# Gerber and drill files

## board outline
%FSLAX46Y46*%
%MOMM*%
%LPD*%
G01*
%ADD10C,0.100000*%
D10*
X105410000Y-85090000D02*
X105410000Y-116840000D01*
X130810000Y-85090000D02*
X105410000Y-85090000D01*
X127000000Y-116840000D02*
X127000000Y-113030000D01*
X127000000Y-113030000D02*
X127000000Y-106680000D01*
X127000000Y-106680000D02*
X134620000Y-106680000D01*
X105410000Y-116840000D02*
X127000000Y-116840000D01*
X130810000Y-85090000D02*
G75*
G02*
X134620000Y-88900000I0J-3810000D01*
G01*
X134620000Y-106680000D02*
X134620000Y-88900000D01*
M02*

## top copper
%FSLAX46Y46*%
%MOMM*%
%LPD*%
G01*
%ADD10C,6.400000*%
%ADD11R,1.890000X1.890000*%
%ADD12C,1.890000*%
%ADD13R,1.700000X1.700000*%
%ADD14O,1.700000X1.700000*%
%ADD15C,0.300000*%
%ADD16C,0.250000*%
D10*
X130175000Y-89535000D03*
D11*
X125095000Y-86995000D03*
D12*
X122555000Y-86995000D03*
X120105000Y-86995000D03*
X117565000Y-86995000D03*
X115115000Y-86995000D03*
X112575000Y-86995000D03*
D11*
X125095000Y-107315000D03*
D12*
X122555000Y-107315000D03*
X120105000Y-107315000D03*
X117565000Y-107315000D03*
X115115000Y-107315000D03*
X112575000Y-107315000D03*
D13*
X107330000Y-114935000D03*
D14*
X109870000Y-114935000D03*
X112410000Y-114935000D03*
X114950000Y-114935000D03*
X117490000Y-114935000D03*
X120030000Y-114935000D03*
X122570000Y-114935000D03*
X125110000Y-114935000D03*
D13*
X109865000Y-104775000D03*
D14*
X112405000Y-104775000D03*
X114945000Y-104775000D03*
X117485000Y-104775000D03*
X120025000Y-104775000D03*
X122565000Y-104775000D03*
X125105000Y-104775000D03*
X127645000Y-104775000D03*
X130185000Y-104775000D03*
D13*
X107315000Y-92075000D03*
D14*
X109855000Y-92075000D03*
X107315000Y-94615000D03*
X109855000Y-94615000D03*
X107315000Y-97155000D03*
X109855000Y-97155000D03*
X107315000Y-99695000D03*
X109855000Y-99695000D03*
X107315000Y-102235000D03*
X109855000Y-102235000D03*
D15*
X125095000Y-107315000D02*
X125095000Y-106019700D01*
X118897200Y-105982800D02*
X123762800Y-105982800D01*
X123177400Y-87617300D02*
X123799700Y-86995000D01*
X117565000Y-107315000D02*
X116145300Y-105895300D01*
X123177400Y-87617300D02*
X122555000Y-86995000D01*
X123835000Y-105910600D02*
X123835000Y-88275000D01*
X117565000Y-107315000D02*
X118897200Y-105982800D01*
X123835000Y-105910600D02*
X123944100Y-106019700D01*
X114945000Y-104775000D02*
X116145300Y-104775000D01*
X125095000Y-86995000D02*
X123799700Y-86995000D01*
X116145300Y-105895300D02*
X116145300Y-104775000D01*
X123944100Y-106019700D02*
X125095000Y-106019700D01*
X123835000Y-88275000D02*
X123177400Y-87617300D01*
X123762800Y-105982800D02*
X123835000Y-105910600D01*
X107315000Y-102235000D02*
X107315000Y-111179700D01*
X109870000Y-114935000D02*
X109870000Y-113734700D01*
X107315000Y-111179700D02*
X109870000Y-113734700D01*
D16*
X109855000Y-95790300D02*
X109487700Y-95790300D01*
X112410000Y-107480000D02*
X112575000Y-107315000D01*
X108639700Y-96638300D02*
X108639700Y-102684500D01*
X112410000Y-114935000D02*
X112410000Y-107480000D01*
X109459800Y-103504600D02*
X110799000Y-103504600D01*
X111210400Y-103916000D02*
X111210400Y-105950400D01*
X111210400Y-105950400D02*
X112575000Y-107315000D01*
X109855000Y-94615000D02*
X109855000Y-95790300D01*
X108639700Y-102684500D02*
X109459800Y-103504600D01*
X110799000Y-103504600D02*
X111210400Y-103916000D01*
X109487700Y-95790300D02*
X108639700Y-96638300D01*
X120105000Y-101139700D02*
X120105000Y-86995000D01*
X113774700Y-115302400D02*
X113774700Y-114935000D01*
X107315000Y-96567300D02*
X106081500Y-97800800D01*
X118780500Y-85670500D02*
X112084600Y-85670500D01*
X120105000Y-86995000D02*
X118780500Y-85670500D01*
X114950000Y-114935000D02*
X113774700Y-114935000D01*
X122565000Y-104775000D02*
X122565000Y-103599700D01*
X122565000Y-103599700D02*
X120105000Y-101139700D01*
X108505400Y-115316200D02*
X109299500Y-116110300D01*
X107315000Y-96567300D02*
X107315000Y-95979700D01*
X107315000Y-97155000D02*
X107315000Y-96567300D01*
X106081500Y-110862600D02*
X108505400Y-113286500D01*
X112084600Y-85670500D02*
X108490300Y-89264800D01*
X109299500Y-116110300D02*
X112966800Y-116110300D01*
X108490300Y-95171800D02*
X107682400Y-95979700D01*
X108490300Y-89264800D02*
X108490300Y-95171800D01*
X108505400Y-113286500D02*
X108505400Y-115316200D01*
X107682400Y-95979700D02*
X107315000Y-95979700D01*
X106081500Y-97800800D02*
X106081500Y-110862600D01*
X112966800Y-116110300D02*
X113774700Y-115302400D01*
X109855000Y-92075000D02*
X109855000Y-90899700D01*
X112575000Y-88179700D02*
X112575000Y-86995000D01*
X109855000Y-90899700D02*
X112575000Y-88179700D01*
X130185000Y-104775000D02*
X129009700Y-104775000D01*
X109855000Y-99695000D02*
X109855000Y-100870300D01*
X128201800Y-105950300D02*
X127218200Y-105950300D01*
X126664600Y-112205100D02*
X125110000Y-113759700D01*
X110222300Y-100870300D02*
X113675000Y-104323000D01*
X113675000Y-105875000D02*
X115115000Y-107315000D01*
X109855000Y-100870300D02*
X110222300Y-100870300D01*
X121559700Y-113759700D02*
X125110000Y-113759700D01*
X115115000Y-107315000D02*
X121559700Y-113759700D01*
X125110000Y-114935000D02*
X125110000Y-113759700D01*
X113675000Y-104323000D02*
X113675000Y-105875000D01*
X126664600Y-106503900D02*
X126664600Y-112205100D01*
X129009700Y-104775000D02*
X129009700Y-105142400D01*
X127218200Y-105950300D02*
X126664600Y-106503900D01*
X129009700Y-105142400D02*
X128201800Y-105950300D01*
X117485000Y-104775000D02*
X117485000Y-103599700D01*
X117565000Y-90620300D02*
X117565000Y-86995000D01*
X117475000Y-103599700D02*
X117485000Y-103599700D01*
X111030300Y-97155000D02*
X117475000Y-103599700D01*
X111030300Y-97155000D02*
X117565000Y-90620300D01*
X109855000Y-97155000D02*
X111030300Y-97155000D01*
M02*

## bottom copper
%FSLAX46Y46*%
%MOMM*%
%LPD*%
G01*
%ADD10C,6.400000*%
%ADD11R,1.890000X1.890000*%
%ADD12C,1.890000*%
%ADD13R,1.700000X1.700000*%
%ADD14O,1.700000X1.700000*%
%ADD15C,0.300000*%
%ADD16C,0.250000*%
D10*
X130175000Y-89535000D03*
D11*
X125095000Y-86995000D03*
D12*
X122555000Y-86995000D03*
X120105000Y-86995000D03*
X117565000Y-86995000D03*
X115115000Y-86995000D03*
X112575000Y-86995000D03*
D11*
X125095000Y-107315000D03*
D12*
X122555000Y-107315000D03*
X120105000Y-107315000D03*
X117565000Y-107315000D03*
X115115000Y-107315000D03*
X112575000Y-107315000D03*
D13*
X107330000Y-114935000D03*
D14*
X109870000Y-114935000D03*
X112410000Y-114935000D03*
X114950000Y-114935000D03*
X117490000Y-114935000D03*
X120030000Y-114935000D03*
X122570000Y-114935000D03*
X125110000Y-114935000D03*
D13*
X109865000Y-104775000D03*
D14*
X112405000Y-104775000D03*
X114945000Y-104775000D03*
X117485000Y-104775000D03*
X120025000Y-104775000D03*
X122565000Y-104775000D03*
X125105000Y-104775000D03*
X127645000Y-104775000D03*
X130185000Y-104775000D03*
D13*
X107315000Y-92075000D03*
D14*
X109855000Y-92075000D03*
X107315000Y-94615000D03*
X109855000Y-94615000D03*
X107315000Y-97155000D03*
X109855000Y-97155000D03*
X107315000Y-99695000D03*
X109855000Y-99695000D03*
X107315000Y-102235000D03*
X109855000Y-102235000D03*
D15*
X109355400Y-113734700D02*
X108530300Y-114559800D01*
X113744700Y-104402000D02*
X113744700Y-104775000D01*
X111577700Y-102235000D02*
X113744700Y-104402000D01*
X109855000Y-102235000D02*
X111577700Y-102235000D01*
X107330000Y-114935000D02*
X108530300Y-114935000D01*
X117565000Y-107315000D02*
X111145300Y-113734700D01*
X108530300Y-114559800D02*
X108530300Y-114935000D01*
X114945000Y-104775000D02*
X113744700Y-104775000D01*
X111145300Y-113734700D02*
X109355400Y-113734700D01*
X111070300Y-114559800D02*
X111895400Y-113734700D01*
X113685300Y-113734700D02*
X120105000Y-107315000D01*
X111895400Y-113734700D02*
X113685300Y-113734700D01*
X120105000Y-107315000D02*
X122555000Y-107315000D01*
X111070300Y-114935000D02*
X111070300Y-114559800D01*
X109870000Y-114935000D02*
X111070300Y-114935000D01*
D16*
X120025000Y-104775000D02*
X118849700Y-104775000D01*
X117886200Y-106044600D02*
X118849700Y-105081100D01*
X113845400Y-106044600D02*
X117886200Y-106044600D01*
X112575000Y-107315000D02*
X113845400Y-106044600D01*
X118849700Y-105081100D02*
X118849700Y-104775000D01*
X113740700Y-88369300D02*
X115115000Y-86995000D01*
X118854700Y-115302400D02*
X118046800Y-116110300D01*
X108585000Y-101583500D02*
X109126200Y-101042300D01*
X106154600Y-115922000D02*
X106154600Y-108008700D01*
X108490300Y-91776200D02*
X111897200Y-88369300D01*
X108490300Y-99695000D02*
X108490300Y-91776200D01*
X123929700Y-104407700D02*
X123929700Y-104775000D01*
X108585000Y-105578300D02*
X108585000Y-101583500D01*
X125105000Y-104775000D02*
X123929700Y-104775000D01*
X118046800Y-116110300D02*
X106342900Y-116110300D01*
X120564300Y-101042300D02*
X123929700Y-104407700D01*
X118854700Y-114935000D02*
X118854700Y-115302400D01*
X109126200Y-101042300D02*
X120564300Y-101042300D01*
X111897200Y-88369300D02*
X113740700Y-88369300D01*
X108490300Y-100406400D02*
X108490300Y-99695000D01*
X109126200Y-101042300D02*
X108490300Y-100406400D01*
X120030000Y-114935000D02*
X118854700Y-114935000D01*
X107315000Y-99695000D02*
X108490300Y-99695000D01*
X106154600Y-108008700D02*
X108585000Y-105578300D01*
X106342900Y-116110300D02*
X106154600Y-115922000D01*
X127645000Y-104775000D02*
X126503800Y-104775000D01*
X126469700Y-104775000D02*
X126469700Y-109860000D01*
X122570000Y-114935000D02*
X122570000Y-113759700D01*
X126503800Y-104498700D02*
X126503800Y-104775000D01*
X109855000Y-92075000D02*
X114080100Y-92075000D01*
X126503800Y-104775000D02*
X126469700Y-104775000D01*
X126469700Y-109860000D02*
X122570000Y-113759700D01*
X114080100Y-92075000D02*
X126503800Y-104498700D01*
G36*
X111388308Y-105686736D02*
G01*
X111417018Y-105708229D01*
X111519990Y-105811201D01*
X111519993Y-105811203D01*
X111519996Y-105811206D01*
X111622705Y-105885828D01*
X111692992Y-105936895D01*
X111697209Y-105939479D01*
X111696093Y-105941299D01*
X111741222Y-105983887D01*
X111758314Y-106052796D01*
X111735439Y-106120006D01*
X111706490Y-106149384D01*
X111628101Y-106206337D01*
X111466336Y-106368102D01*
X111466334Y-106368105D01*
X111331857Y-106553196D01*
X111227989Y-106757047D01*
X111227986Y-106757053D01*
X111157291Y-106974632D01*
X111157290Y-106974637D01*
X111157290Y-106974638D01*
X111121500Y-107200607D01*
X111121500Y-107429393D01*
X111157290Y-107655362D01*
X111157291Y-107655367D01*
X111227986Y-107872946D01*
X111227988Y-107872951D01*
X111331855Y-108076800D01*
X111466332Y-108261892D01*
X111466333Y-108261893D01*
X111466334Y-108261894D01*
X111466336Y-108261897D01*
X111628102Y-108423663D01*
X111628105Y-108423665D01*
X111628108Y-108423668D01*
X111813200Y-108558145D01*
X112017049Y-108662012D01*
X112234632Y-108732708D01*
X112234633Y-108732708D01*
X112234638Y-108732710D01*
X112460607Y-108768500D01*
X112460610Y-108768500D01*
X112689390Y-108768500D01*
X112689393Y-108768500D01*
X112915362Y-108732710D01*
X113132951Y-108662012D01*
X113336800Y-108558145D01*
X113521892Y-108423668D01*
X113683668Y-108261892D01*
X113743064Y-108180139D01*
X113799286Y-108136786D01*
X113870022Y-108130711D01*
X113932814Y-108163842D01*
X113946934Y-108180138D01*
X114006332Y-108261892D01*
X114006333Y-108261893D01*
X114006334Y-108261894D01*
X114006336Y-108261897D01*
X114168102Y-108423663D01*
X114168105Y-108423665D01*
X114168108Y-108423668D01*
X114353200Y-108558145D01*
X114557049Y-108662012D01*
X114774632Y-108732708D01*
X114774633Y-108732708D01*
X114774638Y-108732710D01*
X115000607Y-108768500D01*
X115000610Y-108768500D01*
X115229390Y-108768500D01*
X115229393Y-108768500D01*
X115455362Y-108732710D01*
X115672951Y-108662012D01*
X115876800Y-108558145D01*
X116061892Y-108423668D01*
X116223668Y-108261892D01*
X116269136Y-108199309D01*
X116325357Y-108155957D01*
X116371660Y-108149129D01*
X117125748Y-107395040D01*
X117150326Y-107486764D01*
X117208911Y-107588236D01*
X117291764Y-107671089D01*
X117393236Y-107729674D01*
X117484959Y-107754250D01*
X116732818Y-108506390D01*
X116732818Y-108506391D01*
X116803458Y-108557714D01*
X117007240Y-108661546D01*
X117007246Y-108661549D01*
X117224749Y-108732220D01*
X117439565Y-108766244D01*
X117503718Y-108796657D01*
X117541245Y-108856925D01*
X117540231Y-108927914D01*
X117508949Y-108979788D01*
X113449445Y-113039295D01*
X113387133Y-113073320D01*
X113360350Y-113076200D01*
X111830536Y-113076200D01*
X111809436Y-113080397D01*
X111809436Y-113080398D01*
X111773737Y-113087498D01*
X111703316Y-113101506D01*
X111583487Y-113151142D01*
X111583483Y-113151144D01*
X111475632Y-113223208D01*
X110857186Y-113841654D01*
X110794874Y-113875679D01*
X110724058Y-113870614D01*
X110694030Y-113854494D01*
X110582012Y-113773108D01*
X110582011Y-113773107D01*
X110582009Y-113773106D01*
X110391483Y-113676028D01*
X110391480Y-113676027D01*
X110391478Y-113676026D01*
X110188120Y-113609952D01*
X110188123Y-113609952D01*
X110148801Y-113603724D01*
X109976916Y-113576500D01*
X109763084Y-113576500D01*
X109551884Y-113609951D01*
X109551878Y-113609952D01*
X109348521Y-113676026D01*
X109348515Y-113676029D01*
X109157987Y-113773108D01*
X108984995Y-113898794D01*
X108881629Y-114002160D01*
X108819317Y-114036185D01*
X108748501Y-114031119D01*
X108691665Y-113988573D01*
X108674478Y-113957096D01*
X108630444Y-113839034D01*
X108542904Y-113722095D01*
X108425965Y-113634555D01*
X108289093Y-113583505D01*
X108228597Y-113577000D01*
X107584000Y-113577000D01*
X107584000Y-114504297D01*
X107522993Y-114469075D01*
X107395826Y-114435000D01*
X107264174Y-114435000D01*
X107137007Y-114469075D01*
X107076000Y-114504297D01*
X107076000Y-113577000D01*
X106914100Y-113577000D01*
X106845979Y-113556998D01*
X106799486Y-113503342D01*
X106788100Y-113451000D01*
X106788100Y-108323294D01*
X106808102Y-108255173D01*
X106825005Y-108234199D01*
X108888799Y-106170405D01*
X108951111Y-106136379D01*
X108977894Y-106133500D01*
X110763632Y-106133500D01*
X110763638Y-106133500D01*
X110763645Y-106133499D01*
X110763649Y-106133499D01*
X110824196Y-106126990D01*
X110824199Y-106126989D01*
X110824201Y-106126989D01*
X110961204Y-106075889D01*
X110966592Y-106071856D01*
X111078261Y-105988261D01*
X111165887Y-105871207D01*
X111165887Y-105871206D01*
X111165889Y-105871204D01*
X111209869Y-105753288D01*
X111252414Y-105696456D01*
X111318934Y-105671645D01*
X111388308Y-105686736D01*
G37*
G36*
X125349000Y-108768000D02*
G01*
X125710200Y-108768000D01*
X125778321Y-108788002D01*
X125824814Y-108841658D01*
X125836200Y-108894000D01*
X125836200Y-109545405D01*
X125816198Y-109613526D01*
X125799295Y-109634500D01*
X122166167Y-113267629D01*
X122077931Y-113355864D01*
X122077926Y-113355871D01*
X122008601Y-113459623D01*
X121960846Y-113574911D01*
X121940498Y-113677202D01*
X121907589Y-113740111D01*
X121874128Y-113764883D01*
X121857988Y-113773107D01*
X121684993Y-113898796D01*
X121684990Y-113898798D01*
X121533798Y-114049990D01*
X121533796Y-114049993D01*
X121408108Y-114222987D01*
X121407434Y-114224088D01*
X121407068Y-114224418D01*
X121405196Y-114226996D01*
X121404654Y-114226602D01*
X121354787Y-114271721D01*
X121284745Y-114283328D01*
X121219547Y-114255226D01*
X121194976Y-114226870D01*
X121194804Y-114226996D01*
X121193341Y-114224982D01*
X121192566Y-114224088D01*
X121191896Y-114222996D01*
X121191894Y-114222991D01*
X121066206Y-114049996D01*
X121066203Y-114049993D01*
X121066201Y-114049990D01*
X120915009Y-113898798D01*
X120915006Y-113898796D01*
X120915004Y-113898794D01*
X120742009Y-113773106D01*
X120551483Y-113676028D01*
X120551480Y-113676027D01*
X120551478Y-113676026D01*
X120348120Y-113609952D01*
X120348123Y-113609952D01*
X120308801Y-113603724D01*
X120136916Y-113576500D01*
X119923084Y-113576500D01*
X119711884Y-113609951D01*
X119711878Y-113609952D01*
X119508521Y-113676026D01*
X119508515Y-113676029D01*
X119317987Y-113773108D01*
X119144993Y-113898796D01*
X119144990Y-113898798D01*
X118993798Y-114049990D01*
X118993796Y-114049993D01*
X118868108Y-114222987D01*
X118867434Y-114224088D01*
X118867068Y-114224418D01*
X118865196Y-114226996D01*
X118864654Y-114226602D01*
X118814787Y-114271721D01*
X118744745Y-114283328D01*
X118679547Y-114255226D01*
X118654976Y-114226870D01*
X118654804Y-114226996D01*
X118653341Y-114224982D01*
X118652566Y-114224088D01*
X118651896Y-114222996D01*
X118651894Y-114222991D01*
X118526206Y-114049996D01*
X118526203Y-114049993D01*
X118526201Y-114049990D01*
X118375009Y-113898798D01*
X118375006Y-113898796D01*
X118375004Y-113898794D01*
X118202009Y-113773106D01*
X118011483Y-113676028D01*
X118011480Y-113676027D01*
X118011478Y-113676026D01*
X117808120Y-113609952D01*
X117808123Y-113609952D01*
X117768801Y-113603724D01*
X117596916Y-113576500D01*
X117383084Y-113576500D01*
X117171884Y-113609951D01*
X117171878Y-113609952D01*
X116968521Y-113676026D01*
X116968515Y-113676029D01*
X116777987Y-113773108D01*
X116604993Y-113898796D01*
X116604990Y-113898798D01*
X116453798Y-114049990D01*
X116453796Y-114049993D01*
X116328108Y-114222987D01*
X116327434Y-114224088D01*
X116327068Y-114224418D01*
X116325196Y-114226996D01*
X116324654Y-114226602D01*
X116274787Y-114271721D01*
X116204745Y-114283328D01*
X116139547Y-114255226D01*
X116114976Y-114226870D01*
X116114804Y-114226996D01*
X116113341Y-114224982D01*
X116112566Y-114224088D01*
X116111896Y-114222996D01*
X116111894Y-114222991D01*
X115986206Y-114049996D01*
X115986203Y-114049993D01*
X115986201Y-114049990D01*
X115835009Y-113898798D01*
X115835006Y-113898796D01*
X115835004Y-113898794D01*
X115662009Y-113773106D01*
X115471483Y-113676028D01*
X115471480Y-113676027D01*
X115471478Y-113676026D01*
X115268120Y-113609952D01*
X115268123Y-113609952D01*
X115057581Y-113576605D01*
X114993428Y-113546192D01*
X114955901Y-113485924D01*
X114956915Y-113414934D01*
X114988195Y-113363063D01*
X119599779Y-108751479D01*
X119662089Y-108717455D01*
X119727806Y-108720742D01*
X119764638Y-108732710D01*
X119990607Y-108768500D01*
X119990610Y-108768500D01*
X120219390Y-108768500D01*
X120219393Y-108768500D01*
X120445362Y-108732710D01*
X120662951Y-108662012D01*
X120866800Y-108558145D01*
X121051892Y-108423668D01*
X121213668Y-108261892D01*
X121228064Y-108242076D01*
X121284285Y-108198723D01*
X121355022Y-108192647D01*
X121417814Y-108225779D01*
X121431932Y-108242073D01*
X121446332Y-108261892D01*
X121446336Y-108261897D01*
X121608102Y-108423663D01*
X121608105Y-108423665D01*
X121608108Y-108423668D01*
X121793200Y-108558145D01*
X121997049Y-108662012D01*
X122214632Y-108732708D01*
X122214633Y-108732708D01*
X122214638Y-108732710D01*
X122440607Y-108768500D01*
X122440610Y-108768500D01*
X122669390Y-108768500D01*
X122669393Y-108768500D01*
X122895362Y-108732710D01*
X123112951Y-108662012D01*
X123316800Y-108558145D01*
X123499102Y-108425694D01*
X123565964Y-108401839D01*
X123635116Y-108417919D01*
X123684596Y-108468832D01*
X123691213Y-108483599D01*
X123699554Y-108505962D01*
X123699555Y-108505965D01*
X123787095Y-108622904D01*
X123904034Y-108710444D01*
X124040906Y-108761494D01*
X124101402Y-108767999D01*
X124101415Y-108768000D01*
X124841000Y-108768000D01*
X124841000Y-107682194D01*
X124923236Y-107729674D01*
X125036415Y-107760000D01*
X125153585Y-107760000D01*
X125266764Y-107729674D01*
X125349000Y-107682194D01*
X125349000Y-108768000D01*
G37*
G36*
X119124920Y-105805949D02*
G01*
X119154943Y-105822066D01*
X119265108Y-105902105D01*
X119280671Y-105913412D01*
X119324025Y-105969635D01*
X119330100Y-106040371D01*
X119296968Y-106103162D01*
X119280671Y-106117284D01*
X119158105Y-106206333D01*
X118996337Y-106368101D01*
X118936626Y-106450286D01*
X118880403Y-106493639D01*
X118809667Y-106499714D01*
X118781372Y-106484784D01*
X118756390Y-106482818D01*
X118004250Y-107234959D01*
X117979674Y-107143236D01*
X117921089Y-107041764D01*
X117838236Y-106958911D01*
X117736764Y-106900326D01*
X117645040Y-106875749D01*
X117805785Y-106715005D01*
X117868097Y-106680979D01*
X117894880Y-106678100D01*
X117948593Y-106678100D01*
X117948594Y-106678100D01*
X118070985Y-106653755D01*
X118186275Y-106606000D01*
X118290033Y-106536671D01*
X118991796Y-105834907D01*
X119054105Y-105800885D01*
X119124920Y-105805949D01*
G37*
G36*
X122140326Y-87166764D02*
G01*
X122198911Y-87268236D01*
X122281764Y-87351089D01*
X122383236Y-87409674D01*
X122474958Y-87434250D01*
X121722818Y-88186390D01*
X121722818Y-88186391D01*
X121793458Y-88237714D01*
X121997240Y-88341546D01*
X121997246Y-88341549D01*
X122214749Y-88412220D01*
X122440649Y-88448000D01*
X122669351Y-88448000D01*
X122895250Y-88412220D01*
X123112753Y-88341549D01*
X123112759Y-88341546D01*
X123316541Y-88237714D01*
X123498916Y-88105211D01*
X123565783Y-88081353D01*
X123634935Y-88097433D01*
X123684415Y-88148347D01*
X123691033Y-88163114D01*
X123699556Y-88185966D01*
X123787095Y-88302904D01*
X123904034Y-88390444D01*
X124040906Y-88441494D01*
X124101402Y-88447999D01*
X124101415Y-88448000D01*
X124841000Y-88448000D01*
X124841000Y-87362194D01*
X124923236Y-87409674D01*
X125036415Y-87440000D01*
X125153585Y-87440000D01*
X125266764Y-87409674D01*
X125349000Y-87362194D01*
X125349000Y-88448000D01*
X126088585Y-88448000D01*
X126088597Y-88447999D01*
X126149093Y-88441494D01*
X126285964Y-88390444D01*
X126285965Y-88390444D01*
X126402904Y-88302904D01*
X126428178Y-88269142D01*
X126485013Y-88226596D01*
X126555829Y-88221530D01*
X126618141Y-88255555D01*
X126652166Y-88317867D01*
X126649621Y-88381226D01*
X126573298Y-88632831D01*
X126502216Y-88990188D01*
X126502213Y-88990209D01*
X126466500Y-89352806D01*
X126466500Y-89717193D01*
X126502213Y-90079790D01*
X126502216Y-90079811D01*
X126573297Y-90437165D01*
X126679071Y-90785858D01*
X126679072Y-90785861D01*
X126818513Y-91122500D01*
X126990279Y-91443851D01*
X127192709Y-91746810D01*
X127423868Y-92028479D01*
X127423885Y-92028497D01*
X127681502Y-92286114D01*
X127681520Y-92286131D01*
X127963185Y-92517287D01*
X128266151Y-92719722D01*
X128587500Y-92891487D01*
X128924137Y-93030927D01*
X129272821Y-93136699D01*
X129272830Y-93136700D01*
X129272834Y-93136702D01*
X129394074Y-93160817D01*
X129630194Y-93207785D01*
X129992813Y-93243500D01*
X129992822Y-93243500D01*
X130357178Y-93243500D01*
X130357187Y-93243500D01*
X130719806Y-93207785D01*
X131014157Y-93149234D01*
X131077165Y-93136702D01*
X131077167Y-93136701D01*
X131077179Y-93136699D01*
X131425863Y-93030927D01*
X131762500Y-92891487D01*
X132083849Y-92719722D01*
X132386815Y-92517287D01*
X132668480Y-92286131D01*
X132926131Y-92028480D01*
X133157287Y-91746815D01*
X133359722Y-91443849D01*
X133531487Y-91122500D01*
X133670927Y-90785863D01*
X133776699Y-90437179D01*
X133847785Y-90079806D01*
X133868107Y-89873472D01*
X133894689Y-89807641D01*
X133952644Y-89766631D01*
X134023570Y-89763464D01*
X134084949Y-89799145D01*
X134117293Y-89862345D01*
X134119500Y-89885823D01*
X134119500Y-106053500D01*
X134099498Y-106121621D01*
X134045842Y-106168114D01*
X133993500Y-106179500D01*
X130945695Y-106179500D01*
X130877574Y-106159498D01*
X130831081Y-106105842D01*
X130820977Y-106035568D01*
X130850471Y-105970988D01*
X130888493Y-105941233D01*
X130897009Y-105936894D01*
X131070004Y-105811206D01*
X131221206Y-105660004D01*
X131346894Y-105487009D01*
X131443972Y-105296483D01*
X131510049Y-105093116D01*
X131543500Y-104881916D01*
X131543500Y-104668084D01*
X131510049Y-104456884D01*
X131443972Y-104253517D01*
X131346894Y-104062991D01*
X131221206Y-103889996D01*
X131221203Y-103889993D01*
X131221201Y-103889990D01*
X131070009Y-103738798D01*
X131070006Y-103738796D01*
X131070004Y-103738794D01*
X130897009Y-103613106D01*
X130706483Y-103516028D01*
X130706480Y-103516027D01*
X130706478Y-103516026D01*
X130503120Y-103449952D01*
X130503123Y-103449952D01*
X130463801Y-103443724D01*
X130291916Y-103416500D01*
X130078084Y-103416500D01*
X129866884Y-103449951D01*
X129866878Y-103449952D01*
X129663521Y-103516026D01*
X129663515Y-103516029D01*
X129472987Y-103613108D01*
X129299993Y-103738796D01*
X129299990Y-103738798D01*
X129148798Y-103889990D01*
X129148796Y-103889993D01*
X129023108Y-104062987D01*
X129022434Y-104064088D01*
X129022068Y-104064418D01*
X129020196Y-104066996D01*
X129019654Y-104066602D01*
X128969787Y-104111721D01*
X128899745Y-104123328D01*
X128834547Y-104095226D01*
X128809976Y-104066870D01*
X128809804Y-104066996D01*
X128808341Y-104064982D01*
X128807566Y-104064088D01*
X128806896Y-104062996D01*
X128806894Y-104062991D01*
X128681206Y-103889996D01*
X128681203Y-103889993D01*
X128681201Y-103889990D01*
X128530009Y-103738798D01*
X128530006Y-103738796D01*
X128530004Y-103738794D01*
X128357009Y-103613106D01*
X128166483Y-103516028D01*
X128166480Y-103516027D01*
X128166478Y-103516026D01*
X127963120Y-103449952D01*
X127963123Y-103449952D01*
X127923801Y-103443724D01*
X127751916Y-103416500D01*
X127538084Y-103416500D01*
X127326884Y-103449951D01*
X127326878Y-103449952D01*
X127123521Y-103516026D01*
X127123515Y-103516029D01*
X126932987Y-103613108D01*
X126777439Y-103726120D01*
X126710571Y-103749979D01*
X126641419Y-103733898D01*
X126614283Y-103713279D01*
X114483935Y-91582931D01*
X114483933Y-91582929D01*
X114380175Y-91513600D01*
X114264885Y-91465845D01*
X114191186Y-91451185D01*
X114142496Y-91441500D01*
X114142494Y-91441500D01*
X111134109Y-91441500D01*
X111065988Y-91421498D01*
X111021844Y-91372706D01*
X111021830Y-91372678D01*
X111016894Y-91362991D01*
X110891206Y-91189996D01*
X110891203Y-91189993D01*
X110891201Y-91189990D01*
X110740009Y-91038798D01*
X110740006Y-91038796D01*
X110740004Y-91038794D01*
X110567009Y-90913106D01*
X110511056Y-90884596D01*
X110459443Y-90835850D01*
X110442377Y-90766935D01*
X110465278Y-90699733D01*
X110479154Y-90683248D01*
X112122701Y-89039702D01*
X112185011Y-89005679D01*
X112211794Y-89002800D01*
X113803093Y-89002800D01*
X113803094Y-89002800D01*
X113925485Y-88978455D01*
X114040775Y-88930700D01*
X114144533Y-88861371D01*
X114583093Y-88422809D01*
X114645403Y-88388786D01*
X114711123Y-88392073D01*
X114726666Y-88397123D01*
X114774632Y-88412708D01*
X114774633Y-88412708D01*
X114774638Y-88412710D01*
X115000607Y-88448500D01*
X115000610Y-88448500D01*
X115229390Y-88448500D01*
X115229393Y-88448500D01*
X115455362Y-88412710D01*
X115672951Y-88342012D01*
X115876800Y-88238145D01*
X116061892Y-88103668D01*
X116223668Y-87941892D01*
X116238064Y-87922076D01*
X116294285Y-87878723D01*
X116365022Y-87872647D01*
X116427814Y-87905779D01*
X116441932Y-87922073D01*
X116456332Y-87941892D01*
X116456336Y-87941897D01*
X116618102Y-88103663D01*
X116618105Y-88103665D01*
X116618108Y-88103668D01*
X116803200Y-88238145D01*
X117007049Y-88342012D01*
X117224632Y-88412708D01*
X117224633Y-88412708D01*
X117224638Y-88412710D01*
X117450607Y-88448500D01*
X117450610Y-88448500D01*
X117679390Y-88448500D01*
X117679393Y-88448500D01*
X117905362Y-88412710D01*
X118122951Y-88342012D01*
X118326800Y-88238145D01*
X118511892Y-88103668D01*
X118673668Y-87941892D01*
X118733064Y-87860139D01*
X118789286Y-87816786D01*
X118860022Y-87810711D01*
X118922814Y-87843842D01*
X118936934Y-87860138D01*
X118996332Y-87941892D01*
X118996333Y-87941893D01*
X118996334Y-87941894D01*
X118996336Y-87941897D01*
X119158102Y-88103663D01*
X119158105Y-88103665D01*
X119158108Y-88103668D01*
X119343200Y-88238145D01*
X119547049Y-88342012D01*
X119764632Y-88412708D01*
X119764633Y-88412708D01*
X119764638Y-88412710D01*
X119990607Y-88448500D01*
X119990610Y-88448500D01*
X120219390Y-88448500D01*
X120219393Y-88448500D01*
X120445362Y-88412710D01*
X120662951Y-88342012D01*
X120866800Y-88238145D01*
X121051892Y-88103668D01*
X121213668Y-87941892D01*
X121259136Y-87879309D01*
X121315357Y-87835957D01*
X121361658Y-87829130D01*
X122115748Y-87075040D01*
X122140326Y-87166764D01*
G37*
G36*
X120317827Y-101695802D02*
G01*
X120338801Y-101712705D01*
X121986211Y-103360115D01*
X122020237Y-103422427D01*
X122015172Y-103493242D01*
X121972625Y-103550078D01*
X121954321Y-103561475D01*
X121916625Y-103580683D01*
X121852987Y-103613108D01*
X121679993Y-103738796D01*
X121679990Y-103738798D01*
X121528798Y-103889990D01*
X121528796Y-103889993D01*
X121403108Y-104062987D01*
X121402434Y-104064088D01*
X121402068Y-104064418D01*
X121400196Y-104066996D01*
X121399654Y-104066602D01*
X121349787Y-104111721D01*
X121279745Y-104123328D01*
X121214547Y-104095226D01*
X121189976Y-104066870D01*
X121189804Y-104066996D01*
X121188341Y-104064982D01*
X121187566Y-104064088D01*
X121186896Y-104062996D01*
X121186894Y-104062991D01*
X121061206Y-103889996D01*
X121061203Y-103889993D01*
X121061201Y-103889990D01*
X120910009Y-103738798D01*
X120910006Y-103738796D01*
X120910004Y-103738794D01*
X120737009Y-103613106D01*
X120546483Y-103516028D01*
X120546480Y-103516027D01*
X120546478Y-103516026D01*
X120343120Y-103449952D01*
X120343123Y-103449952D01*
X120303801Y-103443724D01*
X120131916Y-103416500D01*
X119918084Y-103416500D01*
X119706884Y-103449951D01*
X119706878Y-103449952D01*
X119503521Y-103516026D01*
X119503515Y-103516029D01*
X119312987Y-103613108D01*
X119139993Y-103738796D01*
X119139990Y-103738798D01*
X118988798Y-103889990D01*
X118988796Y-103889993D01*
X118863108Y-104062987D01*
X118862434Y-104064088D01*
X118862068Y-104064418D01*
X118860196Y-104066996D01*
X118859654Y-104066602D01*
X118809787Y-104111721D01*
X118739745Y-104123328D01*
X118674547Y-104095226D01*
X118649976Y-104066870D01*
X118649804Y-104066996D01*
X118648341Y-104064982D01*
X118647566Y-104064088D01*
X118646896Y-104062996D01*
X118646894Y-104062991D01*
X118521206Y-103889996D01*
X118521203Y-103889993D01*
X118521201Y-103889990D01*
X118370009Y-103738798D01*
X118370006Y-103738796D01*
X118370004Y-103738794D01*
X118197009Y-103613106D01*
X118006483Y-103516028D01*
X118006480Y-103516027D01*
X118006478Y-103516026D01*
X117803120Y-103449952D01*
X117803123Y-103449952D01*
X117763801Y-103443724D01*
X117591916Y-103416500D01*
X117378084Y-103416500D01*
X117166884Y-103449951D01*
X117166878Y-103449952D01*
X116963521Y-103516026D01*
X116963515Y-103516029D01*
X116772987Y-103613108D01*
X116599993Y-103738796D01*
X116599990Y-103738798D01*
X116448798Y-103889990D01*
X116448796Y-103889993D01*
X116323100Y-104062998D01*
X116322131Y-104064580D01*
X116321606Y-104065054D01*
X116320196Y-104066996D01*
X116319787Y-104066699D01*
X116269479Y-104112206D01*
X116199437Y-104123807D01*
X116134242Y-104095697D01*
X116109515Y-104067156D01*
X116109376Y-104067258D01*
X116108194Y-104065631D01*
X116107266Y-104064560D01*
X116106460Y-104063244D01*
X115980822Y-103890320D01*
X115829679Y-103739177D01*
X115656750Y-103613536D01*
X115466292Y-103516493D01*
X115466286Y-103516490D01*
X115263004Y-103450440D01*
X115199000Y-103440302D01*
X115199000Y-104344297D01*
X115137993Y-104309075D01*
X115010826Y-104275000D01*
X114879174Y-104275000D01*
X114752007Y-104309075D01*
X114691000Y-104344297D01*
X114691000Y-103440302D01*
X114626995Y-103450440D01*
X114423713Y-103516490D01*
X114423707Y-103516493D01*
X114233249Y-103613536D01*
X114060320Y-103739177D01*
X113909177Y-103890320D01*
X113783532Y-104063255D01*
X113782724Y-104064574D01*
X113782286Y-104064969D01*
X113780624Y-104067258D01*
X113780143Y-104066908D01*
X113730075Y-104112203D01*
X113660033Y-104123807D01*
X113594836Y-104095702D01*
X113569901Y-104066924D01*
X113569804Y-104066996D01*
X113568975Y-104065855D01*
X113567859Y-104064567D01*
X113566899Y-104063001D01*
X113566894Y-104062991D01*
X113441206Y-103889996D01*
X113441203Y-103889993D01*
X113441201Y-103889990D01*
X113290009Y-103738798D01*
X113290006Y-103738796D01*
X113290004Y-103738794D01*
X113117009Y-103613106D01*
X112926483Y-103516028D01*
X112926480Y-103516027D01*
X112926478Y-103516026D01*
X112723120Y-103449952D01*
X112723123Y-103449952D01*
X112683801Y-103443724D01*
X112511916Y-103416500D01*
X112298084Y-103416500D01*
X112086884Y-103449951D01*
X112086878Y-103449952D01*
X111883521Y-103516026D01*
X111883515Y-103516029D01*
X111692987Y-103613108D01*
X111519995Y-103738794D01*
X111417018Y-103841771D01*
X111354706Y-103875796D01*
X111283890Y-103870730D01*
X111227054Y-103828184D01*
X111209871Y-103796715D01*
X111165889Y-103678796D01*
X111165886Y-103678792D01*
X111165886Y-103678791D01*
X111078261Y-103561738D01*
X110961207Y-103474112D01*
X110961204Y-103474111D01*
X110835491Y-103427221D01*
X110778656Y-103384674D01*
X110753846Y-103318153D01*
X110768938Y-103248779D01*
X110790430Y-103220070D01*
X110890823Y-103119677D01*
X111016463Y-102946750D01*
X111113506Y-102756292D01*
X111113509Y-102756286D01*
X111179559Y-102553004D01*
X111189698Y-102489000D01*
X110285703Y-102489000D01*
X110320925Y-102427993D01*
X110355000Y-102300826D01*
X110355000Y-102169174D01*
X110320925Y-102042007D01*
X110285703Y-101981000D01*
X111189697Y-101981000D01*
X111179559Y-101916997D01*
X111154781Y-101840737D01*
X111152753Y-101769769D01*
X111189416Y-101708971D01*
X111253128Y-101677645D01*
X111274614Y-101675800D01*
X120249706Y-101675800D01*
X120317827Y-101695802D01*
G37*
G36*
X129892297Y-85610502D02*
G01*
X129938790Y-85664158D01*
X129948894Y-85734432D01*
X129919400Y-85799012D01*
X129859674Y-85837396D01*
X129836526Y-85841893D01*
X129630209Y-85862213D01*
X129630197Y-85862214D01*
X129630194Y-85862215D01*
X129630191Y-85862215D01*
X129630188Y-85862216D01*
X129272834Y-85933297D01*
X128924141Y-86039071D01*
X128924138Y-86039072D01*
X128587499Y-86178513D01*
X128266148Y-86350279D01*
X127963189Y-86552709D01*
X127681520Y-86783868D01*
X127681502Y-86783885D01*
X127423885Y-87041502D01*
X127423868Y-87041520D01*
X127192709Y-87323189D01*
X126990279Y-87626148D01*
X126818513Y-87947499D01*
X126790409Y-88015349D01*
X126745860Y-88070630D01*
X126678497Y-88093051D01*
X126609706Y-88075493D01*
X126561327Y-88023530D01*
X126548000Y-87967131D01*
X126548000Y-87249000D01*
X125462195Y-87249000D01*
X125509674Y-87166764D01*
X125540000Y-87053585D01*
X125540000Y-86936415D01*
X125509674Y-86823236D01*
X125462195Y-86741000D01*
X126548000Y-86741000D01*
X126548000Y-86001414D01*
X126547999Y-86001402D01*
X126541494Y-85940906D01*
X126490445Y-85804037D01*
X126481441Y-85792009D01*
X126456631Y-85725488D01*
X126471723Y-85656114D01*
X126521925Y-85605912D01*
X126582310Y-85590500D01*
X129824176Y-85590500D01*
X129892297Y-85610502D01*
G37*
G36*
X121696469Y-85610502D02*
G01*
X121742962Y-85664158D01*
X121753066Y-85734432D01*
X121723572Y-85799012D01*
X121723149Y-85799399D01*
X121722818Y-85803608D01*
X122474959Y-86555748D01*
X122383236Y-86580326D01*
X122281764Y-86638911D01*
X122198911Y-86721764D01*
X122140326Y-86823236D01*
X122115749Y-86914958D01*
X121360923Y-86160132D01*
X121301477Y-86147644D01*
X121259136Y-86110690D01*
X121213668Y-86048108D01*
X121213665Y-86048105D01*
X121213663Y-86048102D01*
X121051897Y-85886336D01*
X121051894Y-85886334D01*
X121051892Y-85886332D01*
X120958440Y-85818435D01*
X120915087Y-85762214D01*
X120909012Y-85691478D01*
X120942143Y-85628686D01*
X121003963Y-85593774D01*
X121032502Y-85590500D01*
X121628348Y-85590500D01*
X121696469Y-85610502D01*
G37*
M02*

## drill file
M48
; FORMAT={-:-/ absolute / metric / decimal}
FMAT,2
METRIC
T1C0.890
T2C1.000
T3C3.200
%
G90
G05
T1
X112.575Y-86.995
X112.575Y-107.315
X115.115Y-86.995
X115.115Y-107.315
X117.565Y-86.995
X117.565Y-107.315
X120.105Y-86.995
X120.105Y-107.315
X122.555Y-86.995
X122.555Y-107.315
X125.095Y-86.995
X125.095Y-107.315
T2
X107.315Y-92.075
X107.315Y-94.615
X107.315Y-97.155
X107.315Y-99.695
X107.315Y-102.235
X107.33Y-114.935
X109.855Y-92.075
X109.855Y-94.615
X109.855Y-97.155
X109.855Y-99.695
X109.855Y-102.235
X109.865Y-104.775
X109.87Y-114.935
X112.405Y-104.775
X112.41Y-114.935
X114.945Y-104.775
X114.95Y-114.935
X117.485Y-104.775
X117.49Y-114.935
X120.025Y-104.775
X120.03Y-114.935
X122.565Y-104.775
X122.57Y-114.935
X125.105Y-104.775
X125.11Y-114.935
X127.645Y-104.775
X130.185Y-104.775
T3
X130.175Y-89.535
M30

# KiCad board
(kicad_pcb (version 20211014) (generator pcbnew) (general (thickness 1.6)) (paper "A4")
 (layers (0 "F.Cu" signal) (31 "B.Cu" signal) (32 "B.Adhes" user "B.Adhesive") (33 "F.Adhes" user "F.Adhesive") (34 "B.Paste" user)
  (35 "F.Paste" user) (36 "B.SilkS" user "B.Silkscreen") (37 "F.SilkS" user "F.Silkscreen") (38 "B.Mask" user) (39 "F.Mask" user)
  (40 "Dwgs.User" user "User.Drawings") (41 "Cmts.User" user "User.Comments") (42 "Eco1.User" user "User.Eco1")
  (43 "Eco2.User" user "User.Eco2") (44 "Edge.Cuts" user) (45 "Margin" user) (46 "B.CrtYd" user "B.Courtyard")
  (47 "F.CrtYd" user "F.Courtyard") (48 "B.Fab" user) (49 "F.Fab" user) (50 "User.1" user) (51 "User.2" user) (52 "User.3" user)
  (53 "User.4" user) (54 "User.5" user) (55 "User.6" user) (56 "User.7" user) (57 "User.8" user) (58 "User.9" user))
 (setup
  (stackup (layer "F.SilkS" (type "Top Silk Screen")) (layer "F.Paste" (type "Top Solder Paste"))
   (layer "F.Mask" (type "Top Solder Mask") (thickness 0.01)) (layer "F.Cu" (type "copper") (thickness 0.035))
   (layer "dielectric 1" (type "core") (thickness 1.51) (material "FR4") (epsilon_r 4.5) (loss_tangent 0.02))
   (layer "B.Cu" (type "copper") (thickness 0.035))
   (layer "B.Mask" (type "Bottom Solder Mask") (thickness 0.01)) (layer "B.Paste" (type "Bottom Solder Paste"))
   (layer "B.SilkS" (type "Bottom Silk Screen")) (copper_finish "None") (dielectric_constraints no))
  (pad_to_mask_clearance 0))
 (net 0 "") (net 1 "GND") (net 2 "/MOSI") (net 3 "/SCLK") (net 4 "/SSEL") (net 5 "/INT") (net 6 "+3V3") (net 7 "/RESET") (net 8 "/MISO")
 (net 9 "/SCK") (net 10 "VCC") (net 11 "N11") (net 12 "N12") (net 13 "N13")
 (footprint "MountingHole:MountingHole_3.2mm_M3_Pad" (layer "F.Cu") (at 130.175 89.535)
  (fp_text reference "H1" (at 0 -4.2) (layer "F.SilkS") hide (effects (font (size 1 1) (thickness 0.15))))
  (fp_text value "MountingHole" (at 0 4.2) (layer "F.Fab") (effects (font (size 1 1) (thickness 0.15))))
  (pad "1" thru_hole circle locked (at 0 0) (size 6.4 6.4) (drill 3.2) (layers *.Cu *.Mask)))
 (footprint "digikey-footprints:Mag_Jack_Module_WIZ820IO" (layer "F.Cu") (at 118.835 97.155 -90)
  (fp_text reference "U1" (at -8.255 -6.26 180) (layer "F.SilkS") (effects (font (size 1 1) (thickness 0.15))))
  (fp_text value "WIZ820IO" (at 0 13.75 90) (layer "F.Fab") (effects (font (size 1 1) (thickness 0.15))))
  (pad "J1-1" thru_hole rect (at -10.16 -6.26 270) (size 1.89 1.89) (drill 0.89) (layers *.Cu *.Mask) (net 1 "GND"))
  (pad "J1-2" thru_hole circle (at -10.16 -3.72 270) (size 1.89 1.89) (drill 0.89) (layers *.Cu *.Mask) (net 1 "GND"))
  (pad "J1-3" thru_hole circle (at -10.16 -1.27 270) (size 1.89 1.89) (drill 0.89) (layers *.Cu *.Mask) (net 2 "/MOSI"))
  (pad "J1-4" thru_hole circle (at -10.16 1.27 270) (size 1.89 1.89) (drill 0.89) (layers *.Cu *.Mask) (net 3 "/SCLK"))
  (pad "J1-5" thru_hole circle (at -10.16 3.72 270) (size 1.89 1.89) (drill 0.89) (layers *.Cu *.Mask) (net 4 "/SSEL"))
  (pad "J1-6" thru_hole circle (at -10.16 6.26 270) (size 1.89 1.89) (drill 0.89) (layers *.Cu *.Mask) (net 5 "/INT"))
  (pad "J2-1" thru_hole rect (at 10.16 -6.26 270) (size 1.89 1.89) (drill 0.89) (layers *.Cu *.Mask) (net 1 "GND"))
  (pad "J2-2" thru_hole circle (at 10.16 -3.72 270) (size 1.89 1.89) (drill 0.89) (layers *.Cu *.Mask) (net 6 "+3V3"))
  (pad "J2-3" thru_hole circle (at 10.16 -1.27 270) (size 1.89 1.89) (drill 0.89) (layers *.Cu *.Mask) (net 6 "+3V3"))
  (pad "J2-4" thru_hole circle (at 10.16 1.27 270) (size 1.89 1.89) (drill 0.89) (layers *.Cu *.Mask) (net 1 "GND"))
  (pad "J2-5" thru_hole circle (at 10.16 3.72 270) (size 1.89 1.89) (drill 0.89) (layers *.Cu *.Mask) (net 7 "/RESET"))
  (pad "J2-6" thru_hole circle (at 10.16 6.26 270) (size 1.89 1.89) (drill 0.89) (layers *.Cu *.Mask) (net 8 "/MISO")))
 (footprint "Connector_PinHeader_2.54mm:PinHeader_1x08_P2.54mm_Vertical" (layer "F.Cu") (at 107.33 114.935 90)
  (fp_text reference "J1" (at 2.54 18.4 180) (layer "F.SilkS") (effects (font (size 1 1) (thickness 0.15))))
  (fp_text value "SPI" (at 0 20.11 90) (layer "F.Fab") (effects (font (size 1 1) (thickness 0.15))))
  (pad "1" thru_hole rect locked (at 0 0 90) (size 1.7 1.7) (drill 1) (layers *.Cu *.Mask) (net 1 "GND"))
  (pad "2" thru_hole oval locked (at 0 2.54 90) (size 1.7 1.7) (drill 1) (layers *.Cu *.Mask) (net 6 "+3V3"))
  (pad "3" thru_hole oval locked (at 0 5.08 90) (size 1.7 1.7) (drill 1) (layers *.Cu *.Mask) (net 8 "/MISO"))
  (pad "4" thru_hole oval locked (at 0 7.62 90) (size 1.7 1.7) (drill 1) (layers *.Cu *.Mask) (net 2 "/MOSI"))
  (pad "5" thru_hole oval locked (at 0 10.16 90) (size 1.7 1.7) (drill 1) (layers *.Cu *.Mask) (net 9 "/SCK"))
  (pad "6" thru_hole oval locked (at 0 12.7 90) (size 1.7 1.7) (drill 1) (layers *.Cu *.Mask) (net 4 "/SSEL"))
  (pad "7" thru_hole oval locked (at 0 15.24 90) (size 1.7 1.7) (drill 1) (layers *.Cu *.Mask) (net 5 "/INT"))
  (pad "8" thru_hole oval locked (at 0 17.78 90) (size 1.7 1.7) (drill 1) (layers *.Cu *.Mask) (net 7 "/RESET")))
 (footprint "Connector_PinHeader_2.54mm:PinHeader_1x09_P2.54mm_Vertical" (layer "F.Cu") (at 109.865 104.775 90)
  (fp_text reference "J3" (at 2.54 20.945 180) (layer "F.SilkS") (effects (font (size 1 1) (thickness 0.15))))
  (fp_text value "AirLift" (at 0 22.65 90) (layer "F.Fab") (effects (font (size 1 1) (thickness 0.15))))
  (pad "1" thru_hole rect locked (at 0 0 90) (size 1.7 1.7) (drill 1) (layers *.Cu *.Mask) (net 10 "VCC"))
  (pad "2" thru_hole oval locked (at 0 2.54 90) (size 1.7 1.7) (drill 1) (layers *.Cu *.Mask) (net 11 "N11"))
  (pad "3" thru_hole oval locked (at 0 5.08 90) (size 1.7 1.7) (drill 1) (layers *.Cu *.Mask) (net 1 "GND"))
  (pad "4" thru_hole oval locked (at 0 7.62 90) (size 1.7 1.7) (drill 1) (layers *.Cu *.Mask) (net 3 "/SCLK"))
  (pad "5" thru_hole oval locked (at 0 10.16 90) (size 1.7 1.7) (drill 1) (layers *.Cu *.Mask) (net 8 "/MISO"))
  (pad "6" thru_hole oval locked (at 0 12.7 90) (size 1.7 1.7) (drill 1) (layers *.Cu *.Mask) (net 2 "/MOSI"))
  (pad "7" thru_hole oval locked (at 0 15.24 90) (size 1.7 1.7) (drill 1) (layers *.Cu *.Mask) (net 4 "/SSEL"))
  (pad "8" thru_hole oval locked (at 0 17.78 90) (size 1.7 1.7) (drill 1) (layers *.Cu *.Mask) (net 5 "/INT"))
  (pad "9" thru_hole oval locked (at 0 20.32 90) (size 1.7 1.7) (drill 1) (layers *.Cu *.Mask) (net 7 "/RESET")))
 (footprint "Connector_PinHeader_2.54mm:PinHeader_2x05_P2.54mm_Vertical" (layer "F.Cu") (at 107.315 92.075)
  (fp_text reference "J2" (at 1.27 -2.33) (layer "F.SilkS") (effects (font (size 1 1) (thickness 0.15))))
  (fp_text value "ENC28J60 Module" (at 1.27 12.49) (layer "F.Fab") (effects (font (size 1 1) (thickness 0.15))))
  (pad "1" thru_hole rect locked (at 0 0) (size 1.7 1.7) (drill 1) (layers *.Cu *.Mask) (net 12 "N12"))
  (pad "2" thru_hole oval locked (at 2.54 0) (size 1.7 1.7) (drill 1) (layers *.Cu *.Mask) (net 5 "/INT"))
  (pad "3" thru_hole oval locked (at 0 2.54) (size 1.7 1.7) (drill 1) (layers *.Cu *.Mask) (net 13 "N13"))
  (pad "4" thru_hole oval locked (at 2.54 2.54) (size 1.7 1.7) (drill 1) (layers *.Cu *.Mask) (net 8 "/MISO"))
  (pad "5" thru_hole oval locked (at 0 5.08) (size 1.7 1.7) (drill 1) (layers *.Cu *.Mask) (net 2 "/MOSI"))
  (pad "6" thru_hole oval locked (at 2.54 5.08) (size 1.7 1.7) (drill 1) (layers *.Cu *.Mask) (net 3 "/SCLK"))
  (pad "7" thru_hole oval locked (at 0 7.62) (size 1.7 1.7) (drill 1) (layers *.Cu *.Mask) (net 4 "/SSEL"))
  (pad "8" thru_hole oval locked (at 2.54 7.62) (size 1.7 1.7) (drill 1) (layers *.Cu *.Mask) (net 7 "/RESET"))
  (pad "9" thru_hole oval locked (at 0 10.16) (size 1.7 1.7) (drill 1) (layers *.Cu *.Mask) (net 6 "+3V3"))
  (pad "10" thru_hole oval locked (at 2.54 10.16) (size 1.7 1.7) (drill 1) (layers *.Cu *.Mask) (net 1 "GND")))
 (gr_line (start 105.41 85.09) (end 105.41 116.84) (layer "Edge.Cuts") (width 0.1))
 (gr_line (start 130.81 85.09) (end 105.41 85.09) (layer "Edge.Cuts") (width 0.1))
 (gr_line (start 127 116.84) (end 127 113.03) (layer "Edge.Cuts") (width 0.1))
 (gr_line (start 127 113.03) (end 127 106.68) (layer "Edge.Cuts") (width 0.1))
 (gr_line (start 127 106.68) (end 134.62 106.68) (layer "Edge.Cuts") (width 0.1))
 (gr_line (start 105.41 116.84) (end 127 116.84) (layer "Edge.Cuts") (width 0.1))
 (gr_arc (start 130.81 85.09) (mid 133.504077 86.205923) (end 134.62 88.9) (layer "Edge.Cuts") (width 0.1))
 (gr_line (start 134.62 106.68) (end 134.62 88.9) (layer "Edge.Cuts") (width 0.1))
 (segment (start 125.095 107.315) (end 125.095 106.0197) (width 0.3) (layer "F.Cu") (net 1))
 (segment (start 118.8972 105.9828) (end 123.7628 105.9828) (width 0.3) (layer "F.Cu") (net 1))
 (segment (start 123.1774 87.6173) (end 123.7997 86.995) (width 0.3) (layer "F.Cu") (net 1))
 (segment (start 117.565 107.315) (end 116.1453 105.8953) (width 0.3) (layer "F.Cu") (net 1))
 (segment (start 123.1774 87.6173) (end 122.555 86.995) (width 0.3) (layer "F.Cu") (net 1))
 (segment (start 123.835 105.9106) (end 123.835 88.275) (width 0.3) (layer "F.Cu") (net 1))
 (segment (start 117.565 107.315) (end 118.8972 105.9828) (width 0.3) (layer "F.Cu") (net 1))
 (segment (start 123.835 105.9106) (end 123.9441 106.0197) (width 0.3) (layer "F.Cu") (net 1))
 (segment (start 114.945 104.775) (end 116.1453 104.775) (width 0.3) (layer "F.Cu") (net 1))
 (segment (start 125.095 86.995) (end 123.7997 86.995) (width 0.3) (layer "F.Cu") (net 1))
 (segment (start 116.1453 105.8953) (end 116.1453 104.775) (width 0.3) (layer "F.Cu") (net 1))
 (segment (start 123.9441 106.0197) (end 125.095 106.0197) (width 0.3) (layer "F.Cu") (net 1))
 (segment (start 123.835 88.275) (end 123.1774 87.6173) (width 0.3) (layer "F.Cu") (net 1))
 (segment (start 123.7628 105.9828) (end 123.835 105.9106) (width 0.3) (layer "F.Cu") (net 1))
 (segment (start 109.3554 113.7347) (end 108.5303 114.5598) (width 0.3) (layer "B.Cu") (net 1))
 (segment (start 113.7447 104.402) (end 113.7447 104.775) (width 0.3) (layer "B.Cu") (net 1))
 (segment (start 111.5777 102.235) (end 113.7447 104.402) (width 0.3) (layer "B.Cu") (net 1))
 (segment (start 109.855 102.235) (end 111.5777 102.235) (width 0.3) (layer "B.Cu") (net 1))
 (segment (start 107.33 114.935) (end 108.5303 114.935) (width 0.3) (layer "B.Cu") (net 1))
 (segment (start 117.565 107.315) (end 111.1453 113.7347) (width 0.3) (layer "B.Cu") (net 1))
 (segment (start 108.5303 114.5598) (end 108.5303 114.935) (width 0.3) (layer "B.Cu") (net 1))
 (segment (start 114.945 104.775) (end 113.7447 104.775) (width 0.3) (layer "B.Cu") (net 1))
 (segment (start 111.1453 113.7347) (end 109.3554 113.7347) (width 0.3) (layer "B.Cu") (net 1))
 (segment (start 107.315 102.235) (end 107.315 111.1797) (width 0.3) (layer "F.Cu") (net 6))
 (segment (start 109.87 114.935) (end 109.87 113.7347) (width 0.3) (layer "F.Cu") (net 6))
 (segment (start 107.315 111.1797) (end 109.87 113.7347) (width 0.3) (layer "F.Cu") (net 6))
 (segment (start 111.0703 114.5598) (end 111.8954 113.7347) (width 0.3) (layer "B.Cu") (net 6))
 (segment (start 113.6853 113.7347) (end 120.105 107.315) (width 0.3) (layer "B.Cu") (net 6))
 (segment (start 111.8954 113.7347) (end 113.6853 113.7347) (width 0.3) (layer "B.Cu") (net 6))
 (segment (start 120.105 107.315) (end 122.555 107.315) (width 0.3) (layer "B.Cu") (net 6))
 (segment (start 111.0703 114.935) (end 111.0703 114.5598) (width 0.3) (layer "B.Cu") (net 6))
 (segment (start 109.87 114.935) (end 111.0703 114.935) (width 0.3) (layer "B.Cu") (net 6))
 (segment (start 109.855 95.7903) (end 109.4877 95.7903) (width 0.25) (layer "F.Cu") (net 8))
 (segment (start 112.41 107.48) (end 112.575 107.315) (width 0.25) (layer "F.Cu") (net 8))
 (segment (start 108.6397 96.6383) (end 108.6397 102.6845) (width 0.25) (layer "F.Cu") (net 8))
 (segment (start 112.41 114.935) (end 112.41 107.48) (width 0.25) (layer "F.Cu") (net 8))
 (segment (start 109.4598 103.5046) (end 110.799 103.5046) (width 0.25) (layer "F.Cu") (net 8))
 (segment (start 111.2104 103.916) (end 111.2104 105.9504) (width 0.25) (layer "F.Cu") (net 8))
 (segment (start 111.2104 105.9504) (end 112.575 107.315) (width 0.25) (layer "F.Cu") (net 8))
 (segment (start 109.855 94.615) (end 109.855 95.7903) (width 0.25) (layer "F.Cu") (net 8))
 (segment (start 108.6397 102.6845) (end 109.4598 103.5046) (width 0.25) (layer "F.Cu") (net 8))
 (segment (start 110.799 103.5046) (end 111.2104 103.916) (width 0.25) (layer "F.Cu") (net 8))
 (segment (start 109.4877 95.7903) (end 108.6397 96.6383) (width 0.25) (layer "F.Cu") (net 8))
 (segment (start 120.025 104.775) (end 118.8497 104.775) (width 0.25) (layer "B.Cu") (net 8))
 (segment (start 117.8862 106.0446) (end 118.8497 105.0811) (width 0.25) (layer "B.Cu") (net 8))
 (segment (start 113.8454 106.0446) (end 117.8862 106.0446) (width 0.25) (layer "B.Cu") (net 8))
 (segment (start 112.575 107.315) (end 113.8454 106.0446) (width 0.25) (layer "B.Cu") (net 8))
 (segment (start 118.8497 105.0811) (end 118.8497 104.775) (width 0.25) (layer "B.Cu") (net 8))
 (segment (start 120.105 101.1397) (end 120.105 86.995) (width 0.25) (layer "F.Cu") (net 2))
 (segment (start 113.7747 115.3024) (end 113.7747 114.935) (width 0.25) (layer "F.Cu") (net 2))
 (segment (start 107.315 96.5673) (end 106.0815 97.8008) (width 0.25) (layer "F.Cu") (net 2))
 (segment (start 118.7805 85.6705) (end 112.0846 85.6705) (width 0.25) (layer "F.Cu") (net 2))
 (segment (start 120.105 86.995) (end 118.7805 85.6705) (width 0.25) (layer "F.Cu") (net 2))
 (segment (start 114.95 114.935) (end 113.7747 114.935) (width 0.25) (layer "F.Cu") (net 2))
 (segment (start 122.565 104.775) (end 122.565 103.5997) (width 0.25) (layer "F.Cu") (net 2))
 (segment (start 122.565 103.5997) (end 120.105 101.1397) (width 0.25) (layer "F.Cu") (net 2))
 (segment (start 108.5054 115.3162) (end 109.2995 116.1103) (width 0.25) (layer "F.Cu") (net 2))
 (segment (start 107.315 96.5673) (end 107.315 95.9797) (width 0.25) (layer "F.Cu") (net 2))
 (segment (start 107.315 97.155) (end 107.315 96.5673) (width 0.25) (layer "F.Cu") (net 2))
 (segment (start 106.0815 110.8626) (end 108.5054 113.2865) (width 0.25) (layer "F.Cu") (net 2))
 (segment (start 112.0846 85.6705) (end 108.4903 89.2648) (width 0.25) (layer "F.Cu") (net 2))
 (segment (start 109.2995 116.1103) (end 112.9668 116.1103) (width 0.25) (layer "F.Cu") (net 2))
 (segment (start 108.4903 95.1718) (end 107.6824 95.9797) (width 0.25) (layer "F.Cu") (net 2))
 (segment (start 108.4903 89.2648) (end 108.4903 95.1718) (width 0.25) (layer "F.Cu") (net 2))
 (segment (start 108.5054 113.2865) (end 108.5054 115.3162) (width 0.25) (layer "F.Cu") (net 2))
 (segment (start 107.6824 95.9797) (end 107.315 95.9797) (width 0.25) (layer "F.Cu") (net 2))
 (segment (start 106.0815 97.8008) (end 106.0815 110.8626) (width 0.25) (layer "F.Cu") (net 2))
 (segment (start 112.9668 116.1103) (end 113.7747 115.3024) (width 0.25) (layer "F.Cu") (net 2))
 (segment (start 113.7407 88.3693) (end 115.115 86.995) (width 0.25) (layer "B.Cu") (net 4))
 (segment (start 118.8547 115.3024) (end 118.0468 116.1103) (width 0.25) (layer "B.Cu") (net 4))
 (segment (start 108.585 101.5835) (end 109.1262 101.0423) (width 0.25) (layer "B.Cu") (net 4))
 (segment (start 106.1546 115.922) (end 106.1546 108.0087) (width 0.25) (layer "B.Cu") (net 4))
 (segment (start 108.4903 91.7762) (end 111.8972 88.3693) (width 0.25) (layer "B.Cu") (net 4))
 (segment (start 108.4903 99.695) (end 108.4903 91.7762) (width 0.25) (layer "B.Cu") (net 4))
 (segment (start 123.9297 104.4077) (end 123.9297 104.775) (width 0.25) (layer "B.Cu") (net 4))
 (segment (start 108.585 105.5783) (end 108.585 101.5835) (width 0.25) (layer "B.Cu") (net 4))
 (segment (start 125.105 104.775) (end 123.9297 104.775) (width 0.25) (layer "B.Cu") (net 4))
 (segment (start 118.0468 116.1103) (end 106.3429 116.1103) (width 0.25) (layer "B.Cu") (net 4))
 (segment (start 120.5643 101.0423) (end 123.9297 104.4077) (width 0.25) (layer "B.Cu") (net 4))
 (segment (start 118.8547 114.935) (end 118.8547 115.3024) (width 0.25) (layer "B.Cu") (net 4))
 (segment (start 109.1262 101.0423) (end 120.5643 101.0423) (width 0.25) (layer "B.Cu") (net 4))
 (segment (start 111.8972 88.3693) (end 113.7407 88.3693) (width 0.25) (layer "B.Cu") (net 4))
 (segment (start 108.4903 100.4064) (end 108.4903 99.695) (width 0.25) (layer "B.Cu") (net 4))
 (segment (start 109.1262 101.0423) (end 108.4903 100.4064) (width 0.25) (layer "B.Cu") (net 4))
 (segment (start 120.03 114.935) (end 118.8547 114.935) (width 0.25) (layer "B.Cu") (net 4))
 (segment (start 107.315 99.695) (end 108.4903 99.695) (width 0.25) (layer "B.Cu") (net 4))
 (segment (start 106.1546 108.0087) (end 108.585 105.5783) (width 0.25) (layer "B.Cu") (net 4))
 (segment (start 106.3429 116.1103) (end 106.1546 115.922) (width 0.25) (layer "B.Cu") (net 4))
 (segment (start 109.855 92.075) (end 109.855 90.8997) (width 0.25) (layer "F.Cu") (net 5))
 (segment (start 112.575 88.1797) (end 112.575 86.995) (width 0.25) (layer "F.Cu") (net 5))
 (segment (start 109.855 90.8997) (end 112.575 88.1797) (width 0.25) (layer "F.Cu") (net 5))
 (segment (start 127.645 104.775) (end 126.5038 104.775) (width 0.25) (layer "B.Cu") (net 5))
 (segment (start 126.4697 104.775) (end 126.4697 109.86) (width 0.25) (layer "B.Cu") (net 5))
 (segment (start 122.57 114.935) (end 122.57 113.7597) (width 0.25) (layer "B.Cu") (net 5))
 (segment (start 126.5038 104.4987) (end 126.5038 104.775) (width 0.25) (layer "B.Cu") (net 5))
 (segment (start 109.855 92.075) (end 114.0801 92.075) (width 0.25) (layer "B.Cu") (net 5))
 (segment (start 126.5038 104.775) (end 126.4697 104.775) (width 0.25) (layer "B.Cu") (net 5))
 (segment (start 126.4697 109.86) (end 122.57 113.7597) (width 0.25) (layer "B.Cu") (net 5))
 (segment (start 114.0801 92.075) (end 126.5038 104.4987) (width 0.25) (layer "B.Cu") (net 5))
 (segment (start 130.185 104.775) (end 129.0097 104.775) (width 0.25) (layer "F.Cu") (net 7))
 (segment (start 109.855 99.695) (end 109.855 100.8703) (width 0.25) (layer "F.Cu") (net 7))
 (segment (start 128.2018 105.9503) (end 127.2182 105.9503) (width 0.25) (layer "F.Cu") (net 7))
 (segment (start 126.6646 112.2051) (end 125.11 113.7597) (width 0.25) (layer "F.Cu") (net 7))
 (segment (start 110.2223 100.8703) (end 113.675 104.323) (width 0.25) (layer "F.Cu") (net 7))
 (segment (start 113.675 105.875) (end 115.115 107.315) (width 0.25) (layer "F.Cu") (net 7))
 (segment (start 109.855 100.8703) (end 110.2223 100.8703) (width 0.25) (layer "F.Cu") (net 7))
 (segment (start 121.5597 113.7597) (end 125.11 113.7597) (width 0.25) (layer "F.Cu") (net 7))
 (segment (start 115.115 107.315) (end 121.5597 113.7597) (width 0.25) (layer "F.Cu") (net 7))
 (segment (start 125.11 114.935) (end 125.11 113.7597) (width 0.25) (layer "F.Cu") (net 7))
 (segment (start 113.675 104.323) (end 113.675 105.875) (width 0.25) (layer "F.Cu") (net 7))
 (segment (start 126.6646 106.5039) (end 126.6646 112.2051) (width 0.25) (layer "F.Cu") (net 7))
 (segment (start 129.0097 104.775) (end 129.0097 105.1424) (width 0.25) (layer "F.Cu") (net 7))
 (segment (start 127.2182 105.9503) (end 126.6646 106.5039) (width 0.25) (layer "F.Cu") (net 7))
 (segment (start 129.0097 105.1424) (end 128.2018 105.9503) (width 0.25) (layer "F.Cu") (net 7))
 (segment (start 117.485 104.775) (end 117.485 103.5997) (width 0.25) (layer "F.Cu") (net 3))
 (segment (start 117.565 90.6203) (end 117.565 86.995) (width 0.25) (layer "F.Cu") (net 3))
 (segment (start 117.475 103.5997) (end 117.485 103.5997) (width 0.25) (layer "F.Cu") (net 3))
 (segment (start 111.0303 97.155) (end 117.475 103.5997) (width 0.25) (layer "F.Cu") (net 3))
 (segment (start 111.0303 97.155) (end 117.565 90.6203) (width 0.25) (layer "F.Cu") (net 3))
 (segment (start 109.855 97.155) (end 111.0303 97.155) (width 0.25) (layer "F.Cu") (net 3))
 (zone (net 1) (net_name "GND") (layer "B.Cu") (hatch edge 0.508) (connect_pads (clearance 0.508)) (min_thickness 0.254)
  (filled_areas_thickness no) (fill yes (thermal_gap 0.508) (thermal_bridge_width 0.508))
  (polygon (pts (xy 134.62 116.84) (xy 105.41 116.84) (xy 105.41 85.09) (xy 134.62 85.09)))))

